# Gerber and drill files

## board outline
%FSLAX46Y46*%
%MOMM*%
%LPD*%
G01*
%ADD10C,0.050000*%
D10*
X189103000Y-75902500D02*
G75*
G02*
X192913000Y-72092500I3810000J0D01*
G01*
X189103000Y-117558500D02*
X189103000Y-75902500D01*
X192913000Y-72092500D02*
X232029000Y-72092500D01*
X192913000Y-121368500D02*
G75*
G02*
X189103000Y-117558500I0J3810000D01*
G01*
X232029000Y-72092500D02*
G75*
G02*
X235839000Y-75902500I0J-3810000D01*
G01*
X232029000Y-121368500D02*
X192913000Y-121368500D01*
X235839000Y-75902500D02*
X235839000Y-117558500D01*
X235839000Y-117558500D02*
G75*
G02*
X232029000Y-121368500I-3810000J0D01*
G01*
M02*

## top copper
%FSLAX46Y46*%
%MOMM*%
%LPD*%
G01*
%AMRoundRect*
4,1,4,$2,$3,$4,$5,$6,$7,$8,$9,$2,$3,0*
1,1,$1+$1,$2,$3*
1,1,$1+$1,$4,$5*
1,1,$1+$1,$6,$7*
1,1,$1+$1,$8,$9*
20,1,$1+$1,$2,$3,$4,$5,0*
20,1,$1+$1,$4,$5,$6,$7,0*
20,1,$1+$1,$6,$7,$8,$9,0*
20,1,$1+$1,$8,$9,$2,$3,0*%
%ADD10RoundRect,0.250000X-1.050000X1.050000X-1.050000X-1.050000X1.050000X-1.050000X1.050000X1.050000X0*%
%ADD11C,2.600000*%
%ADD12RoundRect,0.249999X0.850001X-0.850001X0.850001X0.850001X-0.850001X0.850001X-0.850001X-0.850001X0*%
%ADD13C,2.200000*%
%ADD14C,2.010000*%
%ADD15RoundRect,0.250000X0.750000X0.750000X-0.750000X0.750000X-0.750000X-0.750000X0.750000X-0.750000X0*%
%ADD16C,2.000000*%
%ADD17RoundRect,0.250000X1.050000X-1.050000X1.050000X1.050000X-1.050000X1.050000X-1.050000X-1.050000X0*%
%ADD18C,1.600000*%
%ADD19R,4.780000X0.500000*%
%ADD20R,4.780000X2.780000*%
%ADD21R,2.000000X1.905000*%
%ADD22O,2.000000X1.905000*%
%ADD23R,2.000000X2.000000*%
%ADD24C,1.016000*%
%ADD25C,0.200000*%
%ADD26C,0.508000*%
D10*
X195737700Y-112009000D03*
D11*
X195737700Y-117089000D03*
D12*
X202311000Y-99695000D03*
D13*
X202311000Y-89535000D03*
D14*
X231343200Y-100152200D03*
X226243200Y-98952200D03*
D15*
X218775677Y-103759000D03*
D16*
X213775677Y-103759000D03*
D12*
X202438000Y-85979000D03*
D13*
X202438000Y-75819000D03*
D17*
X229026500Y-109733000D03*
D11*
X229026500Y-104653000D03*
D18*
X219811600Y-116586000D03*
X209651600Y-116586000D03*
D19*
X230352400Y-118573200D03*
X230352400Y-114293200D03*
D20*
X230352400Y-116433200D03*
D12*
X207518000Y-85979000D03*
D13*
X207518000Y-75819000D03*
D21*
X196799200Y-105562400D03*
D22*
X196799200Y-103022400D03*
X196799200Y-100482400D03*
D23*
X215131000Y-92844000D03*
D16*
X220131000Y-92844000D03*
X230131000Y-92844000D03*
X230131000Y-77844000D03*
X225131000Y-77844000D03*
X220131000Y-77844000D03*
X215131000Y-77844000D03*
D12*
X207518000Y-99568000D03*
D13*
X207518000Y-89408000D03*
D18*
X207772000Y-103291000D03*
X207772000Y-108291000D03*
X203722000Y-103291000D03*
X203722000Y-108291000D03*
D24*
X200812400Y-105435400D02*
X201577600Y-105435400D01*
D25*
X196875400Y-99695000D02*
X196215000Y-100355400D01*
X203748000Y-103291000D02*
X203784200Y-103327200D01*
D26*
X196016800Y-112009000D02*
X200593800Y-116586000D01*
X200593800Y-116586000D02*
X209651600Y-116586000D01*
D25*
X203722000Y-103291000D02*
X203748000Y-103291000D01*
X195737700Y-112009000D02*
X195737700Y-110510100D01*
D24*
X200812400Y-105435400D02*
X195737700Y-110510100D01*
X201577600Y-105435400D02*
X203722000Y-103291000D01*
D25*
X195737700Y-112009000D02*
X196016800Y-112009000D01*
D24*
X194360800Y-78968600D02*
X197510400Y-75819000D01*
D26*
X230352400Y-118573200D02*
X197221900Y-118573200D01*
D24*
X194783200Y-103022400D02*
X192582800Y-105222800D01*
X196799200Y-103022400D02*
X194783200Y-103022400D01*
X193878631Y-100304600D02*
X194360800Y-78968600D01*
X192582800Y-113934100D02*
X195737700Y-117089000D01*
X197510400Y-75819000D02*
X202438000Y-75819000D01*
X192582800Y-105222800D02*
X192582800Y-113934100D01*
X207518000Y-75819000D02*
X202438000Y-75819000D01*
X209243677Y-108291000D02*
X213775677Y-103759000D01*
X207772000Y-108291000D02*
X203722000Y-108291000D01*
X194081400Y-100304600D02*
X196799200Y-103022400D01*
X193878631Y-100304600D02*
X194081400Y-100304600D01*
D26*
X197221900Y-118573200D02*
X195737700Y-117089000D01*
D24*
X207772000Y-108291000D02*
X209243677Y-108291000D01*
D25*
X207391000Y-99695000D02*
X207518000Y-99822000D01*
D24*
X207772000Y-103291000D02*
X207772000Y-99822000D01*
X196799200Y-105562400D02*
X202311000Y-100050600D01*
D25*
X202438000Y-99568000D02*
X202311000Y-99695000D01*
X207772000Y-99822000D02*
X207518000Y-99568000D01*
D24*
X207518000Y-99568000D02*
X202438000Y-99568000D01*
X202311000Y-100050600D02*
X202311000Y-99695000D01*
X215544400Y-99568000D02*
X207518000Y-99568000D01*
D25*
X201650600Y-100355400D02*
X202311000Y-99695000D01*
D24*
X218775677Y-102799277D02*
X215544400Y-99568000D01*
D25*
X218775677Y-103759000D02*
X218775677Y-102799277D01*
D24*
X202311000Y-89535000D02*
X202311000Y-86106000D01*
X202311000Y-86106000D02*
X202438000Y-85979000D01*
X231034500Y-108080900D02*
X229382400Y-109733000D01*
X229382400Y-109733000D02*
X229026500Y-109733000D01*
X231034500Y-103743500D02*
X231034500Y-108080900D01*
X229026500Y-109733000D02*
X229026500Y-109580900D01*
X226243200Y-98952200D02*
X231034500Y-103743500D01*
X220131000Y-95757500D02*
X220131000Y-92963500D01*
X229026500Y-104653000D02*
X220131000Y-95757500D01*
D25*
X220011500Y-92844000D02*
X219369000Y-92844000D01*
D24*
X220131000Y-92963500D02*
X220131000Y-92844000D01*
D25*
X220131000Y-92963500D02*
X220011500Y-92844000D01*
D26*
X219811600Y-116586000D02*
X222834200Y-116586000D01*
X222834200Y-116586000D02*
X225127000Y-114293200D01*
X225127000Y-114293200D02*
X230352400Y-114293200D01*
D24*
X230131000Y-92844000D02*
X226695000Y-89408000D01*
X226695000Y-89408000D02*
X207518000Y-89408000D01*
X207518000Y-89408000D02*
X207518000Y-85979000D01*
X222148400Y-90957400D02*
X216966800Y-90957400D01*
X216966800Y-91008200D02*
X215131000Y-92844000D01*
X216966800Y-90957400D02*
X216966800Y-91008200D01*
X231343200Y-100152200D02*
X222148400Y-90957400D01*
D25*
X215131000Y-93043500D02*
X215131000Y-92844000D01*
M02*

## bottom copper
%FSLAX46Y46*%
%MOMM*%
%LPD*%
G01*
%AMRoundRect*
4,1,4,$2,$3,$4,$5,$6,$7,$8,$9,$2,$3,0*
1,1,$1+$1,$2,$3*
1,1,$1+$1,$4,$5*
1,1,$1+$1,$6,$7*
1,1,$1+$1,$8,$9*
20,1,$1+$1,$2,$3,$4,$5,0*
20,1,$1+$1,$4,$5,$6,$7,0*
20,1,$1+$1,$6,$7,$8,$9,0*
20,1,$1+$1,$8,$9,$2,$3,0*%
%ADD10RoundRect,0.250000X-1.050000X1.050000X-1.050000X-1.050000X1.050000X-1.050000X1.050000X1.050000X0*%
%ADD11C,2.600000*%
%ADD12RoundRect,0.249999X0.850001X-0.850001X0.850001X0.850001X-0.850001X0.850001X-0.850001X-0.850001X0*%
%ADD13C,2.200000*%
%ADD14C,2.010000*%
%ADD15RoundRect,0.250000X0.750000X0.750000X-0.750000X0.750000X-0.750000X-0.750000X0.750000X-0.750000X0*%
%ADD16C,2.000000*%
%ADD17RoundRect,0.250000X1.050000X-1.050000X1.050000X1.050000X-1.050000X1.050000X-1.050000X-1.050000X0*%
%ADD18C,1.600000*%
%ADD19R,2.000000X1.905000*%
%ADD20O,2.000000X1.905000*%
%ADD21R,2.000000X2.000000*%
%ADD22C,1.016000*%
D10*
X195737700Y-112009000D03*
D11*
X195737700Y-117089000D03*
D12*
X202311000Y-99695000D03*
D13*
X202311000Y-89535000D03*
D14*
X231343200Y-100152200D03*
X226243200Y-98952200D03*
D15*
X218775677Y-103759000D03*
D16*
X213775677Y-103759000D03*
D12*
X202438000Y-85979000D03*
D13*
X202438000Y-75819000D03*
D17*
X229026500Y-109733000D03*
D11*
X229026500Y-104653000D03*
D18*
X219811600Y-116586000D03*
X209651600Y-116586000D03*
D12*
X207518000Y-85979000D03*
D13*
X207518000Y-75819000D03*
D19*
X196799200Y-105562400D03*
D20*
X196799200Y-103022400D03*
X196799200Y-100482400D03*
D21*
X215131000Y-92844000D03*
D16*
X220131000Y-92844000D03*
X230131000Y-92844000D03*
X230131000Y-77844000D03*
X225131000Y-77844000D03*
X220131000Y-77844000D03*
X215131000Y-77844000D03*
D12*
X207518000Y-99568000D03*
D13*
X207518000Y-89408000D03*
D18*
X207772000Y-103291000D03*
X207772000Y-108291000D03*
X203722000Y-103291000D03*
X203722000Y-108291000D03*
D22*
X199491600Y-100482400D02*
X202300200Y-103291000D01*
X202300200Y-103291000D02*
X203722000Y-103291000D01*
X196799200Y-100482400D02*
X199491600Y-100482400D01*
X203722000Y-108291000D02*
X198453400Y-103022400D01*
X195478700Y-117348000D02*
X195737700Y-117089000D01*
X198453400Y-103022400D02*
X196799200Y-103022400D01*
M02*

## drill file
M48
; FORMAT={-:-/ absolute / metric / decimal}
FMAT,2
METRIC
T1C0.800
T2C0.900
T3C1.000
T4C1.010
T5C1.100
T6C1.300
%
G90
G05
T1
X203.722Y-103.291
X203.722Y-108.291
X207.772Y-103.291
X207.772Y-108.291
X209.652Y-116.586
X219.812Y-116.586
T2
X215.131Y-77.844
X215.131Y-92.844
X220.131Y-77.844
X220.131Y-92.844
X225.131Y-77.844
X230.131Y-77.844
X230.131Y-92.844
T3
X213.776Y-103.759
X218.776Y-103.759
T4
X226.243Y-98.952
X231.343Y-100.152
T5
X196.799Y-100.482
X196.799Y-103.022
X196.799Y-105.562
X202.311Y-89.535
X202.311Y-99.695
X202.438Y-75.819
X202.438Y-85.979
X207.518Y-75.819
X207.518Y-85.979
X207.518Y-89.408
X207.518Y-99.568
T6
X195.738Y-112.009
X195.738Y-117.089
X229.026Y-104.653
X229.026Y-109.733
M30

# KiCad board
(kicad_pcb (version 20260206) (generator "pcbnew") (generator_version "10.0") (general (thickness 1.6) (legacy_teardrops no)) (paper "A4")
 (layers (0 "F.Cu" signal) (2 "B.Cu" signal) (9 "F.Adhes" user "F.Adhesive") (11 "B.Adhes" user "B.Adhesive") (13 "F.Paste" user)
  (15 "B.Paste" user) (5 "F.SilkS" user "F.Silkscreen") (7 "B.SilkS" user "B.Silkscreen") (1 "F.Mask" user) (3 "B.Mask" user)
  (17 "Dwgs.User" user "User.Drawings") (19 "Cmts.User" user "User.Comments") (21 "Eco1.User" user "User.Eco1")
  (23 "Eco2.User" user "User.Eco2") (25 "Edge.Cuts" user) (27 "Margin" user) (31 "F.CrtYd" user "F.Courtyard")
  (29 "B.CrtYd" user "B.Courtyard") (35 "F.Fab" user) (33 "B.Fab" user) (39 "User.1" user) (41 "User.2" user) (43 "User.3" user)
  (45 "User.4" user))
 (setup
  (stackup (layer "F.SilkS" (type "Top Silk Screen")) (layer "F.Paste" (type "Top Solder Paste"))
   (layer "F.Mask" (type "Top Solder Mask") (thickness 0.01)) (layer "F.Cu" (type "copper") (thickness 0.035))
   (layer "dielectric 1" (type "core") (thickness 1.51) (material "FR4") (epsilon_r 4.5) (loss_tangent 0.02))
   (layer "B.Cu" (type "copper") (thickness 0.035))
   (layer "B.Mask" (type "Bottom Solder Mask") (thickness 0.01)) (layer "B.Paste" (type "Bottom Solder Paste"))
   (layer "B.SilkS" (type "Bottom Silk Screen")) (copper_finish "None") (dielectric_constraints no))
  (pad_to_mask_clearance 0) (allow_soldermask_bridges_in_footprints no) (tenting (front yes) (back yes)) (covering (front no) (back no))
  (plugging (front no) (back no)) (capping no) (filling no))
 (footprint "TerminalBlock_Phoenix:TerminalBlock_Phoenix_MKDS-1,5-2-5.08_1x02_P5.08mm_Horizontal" (layer "F.Cu") (at 195.7377 112.009 -90)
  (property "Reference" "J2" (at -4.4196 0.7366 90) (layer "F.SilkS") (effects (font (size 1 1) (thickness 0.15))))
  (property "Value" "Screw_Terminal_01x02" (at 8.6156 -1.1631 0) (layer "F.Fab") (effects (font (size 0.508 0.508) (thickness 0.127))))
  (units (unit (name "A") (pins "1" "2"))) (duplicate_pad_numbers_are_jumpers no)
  (pad "1" thru_hole roundrect (at 0 0 270) (size 2.6 2.6) (drill 1.3) (layers "*.Cu" "*.Mask") (remove_unused_layers no)
   (roundrect_rratio 0.096154) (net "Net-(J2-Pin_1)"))
  (pad "2" thru_hole circle (at 5.08 0 270) (size 2.6 2.6) (drill 1.3) (layers "*.Cu" "*.Mask") (remove_unused_layers no) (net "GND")))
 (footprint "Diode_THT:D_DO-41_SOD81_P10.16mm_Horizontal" (layer "F.Cu") (at 202.311 99.695 90)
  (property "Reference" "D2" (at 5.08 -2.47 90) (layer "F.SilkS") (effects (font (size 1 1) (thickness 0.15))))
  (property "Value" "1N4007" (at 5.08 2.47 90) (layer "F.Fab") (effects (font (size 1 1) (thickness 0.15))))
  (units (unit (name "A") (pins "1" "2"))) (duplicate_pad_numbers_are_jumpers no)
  (pad "1" thru_hole roundrect (at 0 0 90) (size 2.2 2.2) (drill 1.1) (layers "*.Cu" "*.Mask") (remove_unused_layers no)
   (roundrect_rratio 0.113636) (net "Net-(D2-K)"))
  (pad "2" thru_hole circle (at 10.16 0 90) (size 2.2 2.2) (drill 1.1) (layers "*.Cu" "*.Mask") (remove_unused_layers no) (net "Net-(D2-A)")))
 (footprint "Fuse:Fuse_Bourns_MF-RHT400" (layer "F.Cu") (at 231.3432 100.1522 180)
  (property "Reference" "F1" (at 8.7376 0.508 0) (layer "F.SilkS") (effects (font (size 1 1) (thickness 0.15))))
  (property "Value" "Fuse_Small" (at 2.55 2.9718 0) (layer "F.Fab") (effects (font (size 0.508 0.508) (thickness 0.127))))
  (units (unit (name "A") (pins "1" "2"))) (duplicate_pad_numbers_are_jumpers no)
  (pad "1" thru_hole circle (at 0 0 180) (size 2.01 2.01) (drill 1.01) (layers "*.Cu" "*.Mask") (remove_unused_layers no)
   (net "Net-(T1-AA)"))
  (pad "2" thru_hole circle (at 5.1 1.2 180) (size 2.01 2.01) (drill 1.01) (layers "*.Cu" "*.Mask") (remove_unused_layers no)
   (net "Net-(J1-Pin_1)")))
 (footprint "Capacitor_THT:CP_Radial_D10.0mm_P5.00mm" (layer "F.Cu") (at 218.775677 103.759 180)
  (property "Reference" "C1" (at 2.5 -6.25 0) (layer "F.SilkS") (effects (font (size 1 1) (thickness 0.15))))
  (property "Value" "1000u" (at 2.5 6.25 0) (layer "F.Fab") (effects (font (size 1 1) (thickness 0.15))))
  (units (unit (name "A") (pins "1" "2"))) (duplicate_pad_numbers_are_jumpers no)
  (pad "1" thru_hole roundrect (at 0 0 180) (size 2 2) (drill 1) (layers "*.Cu" "*.Mask") (remove_unused_layers no) (roundrect_rratio 0.125)
   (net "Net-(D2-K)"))
  (pad "2" thru_hole circle (at 5 0 180) (size 2 2) (drill 1) (layers "*.Cu" "*.Mask") (remove_unused_layers no) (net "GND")))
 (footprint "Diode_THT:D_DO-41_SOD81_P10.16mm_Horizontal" (layer "F.Cu") (at 202.438 85.979 90)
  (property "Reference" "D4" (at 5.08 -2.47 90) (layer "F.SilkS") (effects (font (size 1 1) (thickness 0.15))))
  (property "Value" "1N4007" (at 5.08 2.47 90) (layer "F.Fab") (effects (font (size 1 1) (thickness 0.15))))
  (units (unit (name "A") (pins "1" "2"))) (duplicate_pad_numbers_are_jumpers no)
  (pad "1" thru_hole roundrect (at 0 0 90) (size 2.2 2.2) (drill 1.1) (layers "*.Cu" "*.Mask") (remove_unused_layers no)
   (roundrect_rratio 0.113636) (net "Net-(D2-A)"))
  (pad "2" thru_hole circle (at 10.16 0 90) (size 2.2 2.2) (drill 1.1) (layers "*.Cu" "*.Mask") (remove_unused_layers no) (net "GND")))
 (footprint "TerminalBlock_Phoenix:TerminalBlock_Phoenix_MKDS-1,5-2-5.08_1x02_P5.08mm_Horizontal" (layer "F.Cu") (at 229.0265 109.733 90)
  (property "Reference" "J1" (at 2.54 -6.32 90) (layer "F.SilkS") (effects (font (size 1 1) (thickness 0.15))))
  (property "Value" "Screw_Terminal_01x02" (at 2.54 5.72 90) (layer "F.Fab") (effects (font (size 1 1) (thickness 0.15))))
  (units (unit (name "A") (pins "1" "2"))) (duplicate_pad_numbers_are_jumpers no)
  (pad "1" thru_hole roundrect (at 0 0 90) (size 2.6 2.6) (drill 1.3) (layers "*.Cu" "*.Mask") (remove_unused_layers no)
   (roundrect_rratio 0.096154) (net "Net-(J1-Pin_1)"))
  (pad "2" thru_hole circle (at 5.08 0 90) (size 2.6 2.6) (drill 1.3) (layers "*.Cu" "*.Mask") (remove_unused_layers no)
   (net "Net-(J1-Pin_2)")))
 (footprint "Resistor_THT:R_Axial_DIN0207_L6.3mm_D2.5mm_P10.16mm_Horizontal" (layer "F.Cu") (at 219.8116 116.586 180)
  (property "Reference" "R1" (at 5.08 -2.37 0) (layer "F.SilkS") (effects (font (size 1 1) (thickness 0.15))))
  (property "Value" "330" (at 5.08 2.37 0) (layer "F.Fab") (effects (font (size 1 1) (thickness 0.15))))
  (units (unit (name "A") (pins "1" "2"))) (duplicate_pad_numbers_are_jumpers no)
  (pad "1" thru_hole circle (at 0 0 180) (size 1.6 1.6) (drill 0.8) (layers "*.Cu" "*.Mask") (remove_unused_layers no) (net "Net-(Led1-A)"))
  (pad "2" thru_hole circle (at 10.16 0 180) (size 1.6 1.6) (drill 0.8) (layers "*.Cu" "*.Mask") (remove_unused_layers no)
   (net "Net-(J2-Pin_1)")))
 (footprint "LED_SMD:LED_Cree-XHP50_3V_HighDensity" (layer "F.Cu") (at 230.3524 116.4332 90)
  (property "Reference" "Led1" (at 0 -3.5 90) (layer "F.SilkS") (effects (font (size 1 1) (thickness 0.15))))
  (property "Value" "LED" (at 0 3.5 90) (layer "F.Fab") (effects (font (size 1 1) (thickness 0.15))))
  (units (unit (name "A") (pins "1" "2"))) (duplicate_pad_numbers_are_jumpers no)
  (pad "" smd rect (at -2.14 -1.32 90) (size 0.5 2.14) (layers "F.Paste"))
  (pad "" smd rect (at -2.14 1.32 90) (size 0.5 2.14) (layers "F.Paste"))
  (pad "" smd rect (at -0.61 -1.575 90) (size 0.97 0.8) (layers "F.Paste"))
  (pad "" smd rect (at -0.61 -0.525 90) (size 0.97 0.8) (layers "F.Paste"))
  (pad "" smd rect (at -0.61 0.525 90) (size 0.97 0.8) (layers "F.Paste"))
  (pad "" smd rect (at -0.61 1.575 90) (size 0.97 0.8) (layers "F.Paste"))
  (pad "" smd rect (at 0.61 -1.575 90) (size 0.97 0.8) (layers "F.Paste"))
  (pad "" smd rect (at 0.61 -0.525 90) (size 0.97 0.8) (layers "F.Paste"))
  (pad "" smd rect (at 0.61 0.525 90) (size 0.97 0.8) (layers "F.Paste"))
  (pad "" smd rect (at 0.61 1.575 90) (size 0.97 0.8) (layers "F.Paste"))
  (pad "" smd rect (at 2.14 -1.32 90) (size 0.5 2.14) (layers "F.Paste"))
  (pad "" smd rect (at 2.14 1.32 90) (size 0.5 2.14) (layers "F.Paste"))
  (pad "1" smd rect (at -2.14 0 90) (size 0.5 4.78) (layers "F.Cu" "F.Mask") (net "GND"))
  (pad "2" smd rect (at 2.14 0 90) (size 0.5 4.78) (layers "F.Cu" "F.Mask") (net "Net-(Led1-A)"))
  (pad "3" smd rect (at 0 0 90) (size 2.78 4.78) (layers "F.Cu" "F.Mask")))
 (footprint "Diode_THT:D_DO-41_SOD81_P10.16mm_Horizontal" (layer "F.Cu") (at 207.518 85.979 90)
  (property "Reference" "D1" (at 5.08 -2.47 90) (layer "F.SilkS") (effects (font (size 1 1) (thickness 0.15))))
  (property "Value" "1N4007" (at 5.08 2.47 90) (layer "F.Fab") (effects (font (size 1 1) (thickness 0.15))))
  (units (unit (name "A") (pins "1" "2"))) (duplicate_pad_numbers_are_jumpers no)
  (pad "1" thru_hole roundrect (at 0 0 90) (size 2.2 2.2) (drill 1.1) (layers "*.Cu" "*.Mask") (remove_unused_layers no)
   (roundrect_rratio 0.113636) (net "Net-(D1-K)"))
  (pad "2" thru_hole circle (at 10.16 0 90) (size 2.2 2.2) (drill 1.1) (layers "*.Cu" "*.Mask") (remove_unused_layers no) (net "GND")))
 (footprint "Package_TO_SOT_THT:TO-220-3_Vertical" (layer "F.Cu") (at 196.7992 105.5624 90)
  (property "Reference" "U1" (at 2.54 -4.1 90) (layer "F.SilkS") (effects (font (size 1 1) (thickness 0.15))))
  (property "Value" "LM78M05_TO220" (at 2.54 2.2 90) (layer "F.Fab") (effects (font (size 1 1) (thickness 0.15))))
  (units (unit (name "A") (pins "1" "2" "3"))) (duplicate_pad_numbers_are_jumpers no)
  (pad "1" thru_hole rect (at 0 0 90) (size 1.905 2) (drill 1.1) (layers "*.Cu" "*.Mask") (remove_unused_layers no) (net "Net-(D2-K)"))
  (pad "2" thru_hole oval (at 2.54 0 90) (size 1.905 2) (drill 1.1) (layers "*.Cu" "*.Mask") (remove_unused_layers no) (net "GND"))
  (pad "3" thru_hole oval (at 5.08 0 90) (size 1.905 2) (drill 1.1) (layers "*.Cu" "*.Mask") (remove_unused_layers no)
   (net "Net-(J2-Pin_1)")))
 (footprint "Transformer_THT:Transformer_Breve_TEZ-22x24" (layer "F.Cu") (at 215.131 92.844)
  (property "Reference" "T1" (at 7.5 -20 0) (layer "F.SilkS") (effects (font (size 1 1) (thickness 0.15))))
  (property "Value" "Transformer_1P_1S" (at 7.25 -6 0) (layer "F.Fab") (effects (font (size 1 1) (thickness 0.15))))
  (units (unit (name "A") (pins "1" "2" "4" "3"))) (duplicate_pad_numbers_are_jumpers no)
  (pad "1" thru_hole rect (at 0 0) (size 2 2) (drill 0.9) (layers "*.Cu" "*.Mask") (remove_unused_layers no) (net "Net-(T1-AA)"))
  (pad "2" thru_hole circle (at 5 0) (size 2 2) (drill 0.9) (layers "*.Cu" "*.Mask") (remove_unused_layers no) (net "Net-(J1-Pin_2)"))
  (pad "4" thru_hole circle (at 15 0) (size 2 2) (drill 0.9) (layers "*.Cu" "*.Mask") (remove_unused_layers no) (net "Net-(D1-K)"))
  (pad "5" thru_hole circle (at 15 -15) (size 2 2) (drill 0.9) (layers "*.Cu" "*.Mask") (remove_unused_layers no))
  (pad "6" thru_hole circle (at 10 -15) (size 2 2) (drill 0.9) (layers "*.Cu" "*.Mask") (remove_unused_layers no))
  (pad "7" thru_hole circle (at 5 -15) (size 2 2) (drill 0.9) (layers "*.Cu" "*.Mask") (remove_unused_layers no))
  (pad "8" thru_hole circle (at 0 -15) (size 2 2) (drill 0.9) (layers "*.Cu" "*.Mask") (remove_unused_layers no)))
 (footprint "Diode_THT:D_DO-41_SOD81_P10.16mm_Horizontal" (layer "F.Cu") (at 207.518 99.568 90)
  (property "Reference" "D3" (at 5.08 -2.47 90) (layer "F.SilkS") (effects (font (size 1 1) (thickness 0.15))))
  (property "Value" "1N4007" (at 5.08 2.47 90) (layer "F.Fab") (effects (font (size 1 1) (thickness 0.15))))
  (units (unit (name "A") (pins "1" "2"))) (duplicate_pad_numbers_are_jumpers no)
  (pad "1" thru_hole roundrect (at 0 0 90) (size 2.2 2.2) (drill 1.1) (layers "*.Cu" "*.Mask") (remove_unused_layers no)
   (roundrect_rratio 0.113636) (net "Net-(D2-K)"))
  (pad "2" thru_hole circle (at 10.16 0 90) (size 2.2 2.2) (drill 1.1) (layers "*.Cu" "*.Mask") (remove_unused_layers no) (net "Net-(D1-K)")))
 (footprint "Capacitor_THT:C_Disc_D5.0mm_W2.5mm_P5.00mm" (layer "F.Cu") (at 207.772 103.291 -90)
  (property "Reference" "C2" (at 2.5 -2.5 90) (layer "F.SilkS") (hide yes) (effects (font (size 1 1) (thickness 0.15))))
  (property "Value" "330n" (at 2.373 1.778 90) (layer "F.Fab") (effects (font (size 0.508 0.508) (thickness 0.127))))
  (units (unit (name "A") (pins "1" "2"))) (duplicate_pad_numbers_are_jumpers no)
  (pad "1" thru_hole circle (at 0 0 270) (size 1.6 1.6) (drill 0.8) (layers "*.Cu" "*.Mask") (remove_unused_layers no) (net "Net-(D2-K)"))
  (pad "2" thru_hole circle (at 5 0 270) (size 1.6 1.6) (drill 0.8) (layers "*.Cu" "*.Mask") (remove_unused_layers no) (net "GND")))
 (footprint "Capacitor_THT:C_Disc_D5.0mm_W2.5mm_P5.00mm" (layer "F.Cu") (at 203.722 103.291 -90)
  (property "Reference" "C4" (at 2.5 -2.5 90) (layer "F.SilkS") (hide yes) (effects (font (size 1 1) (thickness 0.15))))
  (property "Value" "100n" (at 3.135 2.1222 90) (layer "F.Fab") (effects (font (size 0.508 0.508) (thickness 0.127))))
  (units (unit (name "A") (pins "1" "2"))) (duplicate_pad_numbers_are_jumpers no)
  (pad "1" thru_hole circle (at 0 0 270) (size 1.6 1.6) (drill 0.8) (layers "*.Cu" "*.Mask") (remove_unused_layers no)
   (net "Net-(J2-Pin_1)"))
  (pad "2" thru_hole circle (at 5 0 270) (size 1.6 1.6) (drill 0.8) (layers "*.Cu" "*.Mask") (remove_unused_layers no) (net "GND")))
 (gr_arc (start 189.103 75.9025) (mid 190.218923 73.208423) (end 192.913 72.0925) (stroke (width 0.05) (type default)) (layer "Edge.Cuts"))
 (gr_line (start 189.103 117.5585) (end 189.103 75.9025) (stroke (width 0.05) (type default)) (layer "Edge.Cuts"))
 (gr_line (start 192.913 72.0925) (end 232.029 72.0925) (stroke (width 0.05) (type default)) (layer "Edge.Cuts"))
 (gr_arc (start 192.913 121.3685) (mid 190.218923 120.252577) (end 189.103 117.5585) (stroke (width 0.05) (type default))
  (layer "Edge.Cuts"))
 (gr_arc (start 232.029 72.0925) (mid 234.723077 73.208423) (end 235.839 75.9025) (stroke (width 0.05) (type default)) (layer "Edge.Cuts"))
 (gr_line (start 232.029 121.3685) (end 192.913 121.3685) (stroke (width 0.05) (type default)) (layer "Edge.Cuts"))
 (gr_line (start 235.839 75.9025) (end 235.839 117.5585) (stroke (width 0.05) (type default)) (layer "Edge.Cuts"))
 (gr_arc (start 235.839 117.5585) (mid 234.723077 120.252577) (end 232.029 121.3685) (stroke (width 0.05) (type default))
  (layer "Edge.Cuts"))
 (segment (start 200.8124 105.4354) (end 201.5776 105.4354) (width 1.016) (layer "F.Cu") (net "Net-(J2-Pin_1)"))
 (segment (start 196.8754 99.695) (end 196.215 100.3554) (width 0.2) (layer "F.Cu") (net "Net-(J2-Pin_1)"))
 (segment (start 203.748 103.291) (end 203.7842 103.3272) (width 0.2) (layer "F.Cu") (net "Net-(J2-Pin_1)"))
 (segment (start 196.0168 112.009) (end 200.5938 116.586) (width 0.508) (layer "F.Cu") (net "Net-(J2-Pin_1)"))
 (segment (start 200.5938 116.586) (end 209.6516 116.586) (width 0.508) (layer "F.Cu") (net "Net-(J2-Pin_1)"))
 (segment (start 203.722 103.291) (end 203.748 103.291) (width 0.2) (layer "F.Cu") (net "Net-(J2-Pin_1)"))
 (segment (start 195.7377 112.009) (end 195.7377 110.5101) (width 0.2) (layer "F.Cu") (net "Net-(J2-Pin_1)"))
 (segment (start 200.8124 105.4354) (end 195.7377 110.5101) (width 1.016) (layer "F.Cu") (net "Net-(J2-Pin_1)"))
 (segment (start 201.5776 105.4354) (end 203.722 103.291) (width 1.016) (layer "F.Cu") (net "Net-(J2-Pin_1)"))
 (segment (start 195.7377 112.009) (end 196.0168 112.009) (width 0.2) (layer "F.Cu") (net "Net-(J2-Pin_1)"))
 (segment (start 199.4916 100.4824) (end 202.3002 103.291) (width 1.016) (layer "B.Cu") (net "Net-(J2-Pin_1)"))
 (segment (start 202.3002 103.291) (end 203.722 103.291) (width 1.016) (layer "B.Cu") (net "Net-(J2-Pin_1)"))
 (segment (start 196.7992 100.4824) (end 199.4916 100.4824) (width 1.016) (layer "B.Cu") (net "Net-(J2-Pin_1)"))
 (segment (start 194.3608 78.9686) (end 197.5104 75.819) (width 1.016) (layer "F.Cu") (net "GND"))
 (segment (start 230.3524 118.5732) (end 197.2219 118.5732) (width 0.508) (layer "F.Cu") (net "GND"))
 (segment (start 194.7832 103.0224) (end 192.5828 105.2228) (width 1.016) (layer "F.Cu") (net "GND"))
 (segment (start 196.7992 103.0224) (end 194.7832 103.0224) (width 1.016) (layer "F.Cu") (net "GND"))
 (segment (start 193.878631 100.3046) (end 194.3608 78.9686) (width 1.016) (layer "F.Cu") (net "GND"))
 (segment (start 192.5828 113.9341) (end 195.7377 117.089) (width 1.016) (layer "F.Cu") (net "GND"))
 (segment (start 197.5104 75.819) (end 202.438 75.819) (width 1.016) (layer "F.Cu") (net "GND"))
 (segment (start 192.5828 105.2228) (end 192.5828 113.9341) (width 1.016) (layer "F.Cu") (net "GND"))
 (segment (start 207.518 75.819) (end 202.438 75.819) (width 1.016) (layer "F.Cu") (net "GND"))
 (segment (start 209.243677 108.291) (end 213.775677 103.759) (width 1.016) (layer "F.Cu") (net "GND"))
 (segment (start 207.772 108.291) (end 203.722 108.291) (width 1.016) (layer "F.Cu") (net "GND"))
 (segment (start 194.0814 100.3046) (end 196.7992 103.0224) (width 1.016) (layer "F.Cu") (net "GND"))
 (segment (start 193.878631 100.3046) (end 194.0814 100.3046) (width 1.016) (layer "F.Cu") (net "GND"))
 (segment (start 197.2219 118.5732) (end 195.7377 117.089) (width 0.508) (layer "F.Cu") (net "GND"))
 (segment (start 207.772 108.291) (end 209.243677 108.291) (width 1.016) (layer "F.Cu") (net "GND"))
 (segment (start 203.722 108.291) (end 198.4534 103.0224) (width 1.016) (layer "B.Cu") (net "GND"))
 (segment (start 195.4787 117.348) (end 195.7377 117.089) (width 1.016) (layer "B.Cu") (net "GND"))
 (segment (start 198.4534 103.0224) (end 196.7992 103.0224) (width 1.016) (layer "B.Cu") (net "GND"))
 (segment (start 207.391 99.695) (end 207.518 99.822) (width 0.2) (layer "F.Cu") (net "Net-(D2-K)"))
 (segment (start 207.772 103.291) (end 207.772 99.822) (width 1.016) (layer "F.Cu") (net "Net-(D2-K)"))
 (segment (start 196.7992 105.5624) (end 202.311 100.0506) (width 1.016) (layer "F.Cu") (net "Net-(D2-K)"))
 (segment (start 202.438 99.568) (end 202.311 99.695) (width 0.2) (layer "F.Cu") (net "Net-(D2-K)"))
 (segment (start 207.772 99.822) (end 207.518 99.568) (width 0.2) (layer "F.Cu") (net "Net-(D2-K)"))
 (segment (start 207.518 99.568) (end 202.438 99.568) (width 1.016) (layer "F.Cu") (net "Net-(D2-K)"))
 (segment (start 202.311 100.0506) (end 202.311 99.695) (width 1.016) (layer "F.Cu") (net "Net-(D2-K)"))
 (segment (start 215.5444 99.568) (end 207.518 99.568) (width 1.016) (layer "F.Cu") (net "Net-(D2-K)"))
 (segment (start 201.6506 100.3554) (end 202.311 99.695) (width 0.2) (layer "F.Cu") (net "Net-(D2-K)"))
 (segment (start 218.775677 102.799277) (end 215.5444 99.568) (width 1.016) (layer "F.Cu") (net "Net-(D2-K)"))
 (segment (start 218.775677 103.759) (end 218.775677 102.799277) (width 0.2) (layer "F.Cu") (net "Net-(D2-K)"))
 (segment (start 202.311 89.535) (end 202.311 86.106) (width 1.016) (layer "F.Cu") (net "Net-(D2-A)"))
 (segment (start 202.311 86.106) (end 202.438 85.979) (width 1.016) (layer "F.Cu") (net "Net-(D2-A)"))
 (segment (start 231.0345 108.0809) (end 229.3824 109.733) (width 1.016) (layer "F.Cu") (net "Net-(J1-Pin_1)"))
 (segment (start 229.3824 109.733) (end 229.0265 109.733) (width 1.016) (layer "F.Cu") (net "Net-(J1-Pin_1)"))
 (segment (start 231.0345 103.7435) (end 231.0345 108.0809) (width 1.016) (layer "F.Cu") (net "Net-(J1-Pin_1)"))
 (segment (start 229.0265 109.733) (end 229.0265 109.5809) (width 1.016) (layer "F.Cu") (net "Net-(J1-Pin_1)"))
 (segment (start 226.2432 98.9522) (end 231.0345 103.7435) (width 1.016) (layer "F.Cu") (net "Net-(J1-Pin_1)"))
 (segment (start 220.131 95.7575) (end 220.131 92.9635) (width 1.016) (layer "F.Cu") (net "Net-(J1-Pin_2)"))
 (segment (start 229.0265 104.653) (end 220.131 95.7575) (width 1.016) (layer "F.Cu") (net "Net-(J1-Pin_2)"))
 (segment (start 220.0115 92.844) (end 219.369 92.844) (width 0.2) (layer "F.Cu") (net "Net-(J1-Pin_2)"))
 (segment (start 220.131 92.9635) (end 220.131 92.844) (width 1.016) (layer "F.Cu") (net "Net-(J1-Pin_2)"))
 (segment (start 220.131 92.9635) (end 220.0115 92.844) (width 0.2) (layer "F.Cu") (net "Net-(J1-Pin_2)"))
 (segment (start 219.8116 116.586) (end 222.8342 116.586) (width 0.508) (layer "F.Cu") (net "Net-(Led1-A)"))
 (segment (start 222.8342 116.586) (end 225.127 114.2932) (width 0.508) (layer "F.Cu") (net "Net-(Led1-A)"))
 (segment (start 225.127 114.2932) (end 230.3524 114.2932) (width 0.508) (layer "F.Cu") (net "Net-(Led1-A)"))
 (segment (start 230.131 92.844) (end 226.695 89.408) (width 1.016) (layer "F.Cu") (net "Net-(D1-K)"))
 (segment (start 226.695 89.408) (end 207.518 89.408) (width 1.016) (layer "F.Cu") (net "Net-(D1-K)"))
 (segment (start 207.518 89.408) (end 207.518 85.979) (width 1.016) (layer "F.Cu") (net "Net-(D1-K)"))
 (segment (start 222.1484 90.9574) (end 216.9668 90.9574) (width 1.016) (layer "F.Cu") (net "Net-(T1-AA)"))
 (segment (start 216.9668 91.0082) (end 215.131 92.844) (width 1.016) (layer "F.Cu") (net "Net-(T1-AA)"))
 (segment (start 216.9668 90.9574) (end 216.9668 91.0082) (width 1.016) (layer "F.Cu") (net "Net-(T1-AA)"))
 (segment (start 231.3432 100.1522) (end 222.1484 90.9574) (width 1.016) (layer "F.Cu") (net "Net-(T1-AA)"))
 (segment (start 215.131 93.0435) (end 215.131 92.844) (width 0.2) (layer "F.Cu") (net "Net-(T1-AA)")))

